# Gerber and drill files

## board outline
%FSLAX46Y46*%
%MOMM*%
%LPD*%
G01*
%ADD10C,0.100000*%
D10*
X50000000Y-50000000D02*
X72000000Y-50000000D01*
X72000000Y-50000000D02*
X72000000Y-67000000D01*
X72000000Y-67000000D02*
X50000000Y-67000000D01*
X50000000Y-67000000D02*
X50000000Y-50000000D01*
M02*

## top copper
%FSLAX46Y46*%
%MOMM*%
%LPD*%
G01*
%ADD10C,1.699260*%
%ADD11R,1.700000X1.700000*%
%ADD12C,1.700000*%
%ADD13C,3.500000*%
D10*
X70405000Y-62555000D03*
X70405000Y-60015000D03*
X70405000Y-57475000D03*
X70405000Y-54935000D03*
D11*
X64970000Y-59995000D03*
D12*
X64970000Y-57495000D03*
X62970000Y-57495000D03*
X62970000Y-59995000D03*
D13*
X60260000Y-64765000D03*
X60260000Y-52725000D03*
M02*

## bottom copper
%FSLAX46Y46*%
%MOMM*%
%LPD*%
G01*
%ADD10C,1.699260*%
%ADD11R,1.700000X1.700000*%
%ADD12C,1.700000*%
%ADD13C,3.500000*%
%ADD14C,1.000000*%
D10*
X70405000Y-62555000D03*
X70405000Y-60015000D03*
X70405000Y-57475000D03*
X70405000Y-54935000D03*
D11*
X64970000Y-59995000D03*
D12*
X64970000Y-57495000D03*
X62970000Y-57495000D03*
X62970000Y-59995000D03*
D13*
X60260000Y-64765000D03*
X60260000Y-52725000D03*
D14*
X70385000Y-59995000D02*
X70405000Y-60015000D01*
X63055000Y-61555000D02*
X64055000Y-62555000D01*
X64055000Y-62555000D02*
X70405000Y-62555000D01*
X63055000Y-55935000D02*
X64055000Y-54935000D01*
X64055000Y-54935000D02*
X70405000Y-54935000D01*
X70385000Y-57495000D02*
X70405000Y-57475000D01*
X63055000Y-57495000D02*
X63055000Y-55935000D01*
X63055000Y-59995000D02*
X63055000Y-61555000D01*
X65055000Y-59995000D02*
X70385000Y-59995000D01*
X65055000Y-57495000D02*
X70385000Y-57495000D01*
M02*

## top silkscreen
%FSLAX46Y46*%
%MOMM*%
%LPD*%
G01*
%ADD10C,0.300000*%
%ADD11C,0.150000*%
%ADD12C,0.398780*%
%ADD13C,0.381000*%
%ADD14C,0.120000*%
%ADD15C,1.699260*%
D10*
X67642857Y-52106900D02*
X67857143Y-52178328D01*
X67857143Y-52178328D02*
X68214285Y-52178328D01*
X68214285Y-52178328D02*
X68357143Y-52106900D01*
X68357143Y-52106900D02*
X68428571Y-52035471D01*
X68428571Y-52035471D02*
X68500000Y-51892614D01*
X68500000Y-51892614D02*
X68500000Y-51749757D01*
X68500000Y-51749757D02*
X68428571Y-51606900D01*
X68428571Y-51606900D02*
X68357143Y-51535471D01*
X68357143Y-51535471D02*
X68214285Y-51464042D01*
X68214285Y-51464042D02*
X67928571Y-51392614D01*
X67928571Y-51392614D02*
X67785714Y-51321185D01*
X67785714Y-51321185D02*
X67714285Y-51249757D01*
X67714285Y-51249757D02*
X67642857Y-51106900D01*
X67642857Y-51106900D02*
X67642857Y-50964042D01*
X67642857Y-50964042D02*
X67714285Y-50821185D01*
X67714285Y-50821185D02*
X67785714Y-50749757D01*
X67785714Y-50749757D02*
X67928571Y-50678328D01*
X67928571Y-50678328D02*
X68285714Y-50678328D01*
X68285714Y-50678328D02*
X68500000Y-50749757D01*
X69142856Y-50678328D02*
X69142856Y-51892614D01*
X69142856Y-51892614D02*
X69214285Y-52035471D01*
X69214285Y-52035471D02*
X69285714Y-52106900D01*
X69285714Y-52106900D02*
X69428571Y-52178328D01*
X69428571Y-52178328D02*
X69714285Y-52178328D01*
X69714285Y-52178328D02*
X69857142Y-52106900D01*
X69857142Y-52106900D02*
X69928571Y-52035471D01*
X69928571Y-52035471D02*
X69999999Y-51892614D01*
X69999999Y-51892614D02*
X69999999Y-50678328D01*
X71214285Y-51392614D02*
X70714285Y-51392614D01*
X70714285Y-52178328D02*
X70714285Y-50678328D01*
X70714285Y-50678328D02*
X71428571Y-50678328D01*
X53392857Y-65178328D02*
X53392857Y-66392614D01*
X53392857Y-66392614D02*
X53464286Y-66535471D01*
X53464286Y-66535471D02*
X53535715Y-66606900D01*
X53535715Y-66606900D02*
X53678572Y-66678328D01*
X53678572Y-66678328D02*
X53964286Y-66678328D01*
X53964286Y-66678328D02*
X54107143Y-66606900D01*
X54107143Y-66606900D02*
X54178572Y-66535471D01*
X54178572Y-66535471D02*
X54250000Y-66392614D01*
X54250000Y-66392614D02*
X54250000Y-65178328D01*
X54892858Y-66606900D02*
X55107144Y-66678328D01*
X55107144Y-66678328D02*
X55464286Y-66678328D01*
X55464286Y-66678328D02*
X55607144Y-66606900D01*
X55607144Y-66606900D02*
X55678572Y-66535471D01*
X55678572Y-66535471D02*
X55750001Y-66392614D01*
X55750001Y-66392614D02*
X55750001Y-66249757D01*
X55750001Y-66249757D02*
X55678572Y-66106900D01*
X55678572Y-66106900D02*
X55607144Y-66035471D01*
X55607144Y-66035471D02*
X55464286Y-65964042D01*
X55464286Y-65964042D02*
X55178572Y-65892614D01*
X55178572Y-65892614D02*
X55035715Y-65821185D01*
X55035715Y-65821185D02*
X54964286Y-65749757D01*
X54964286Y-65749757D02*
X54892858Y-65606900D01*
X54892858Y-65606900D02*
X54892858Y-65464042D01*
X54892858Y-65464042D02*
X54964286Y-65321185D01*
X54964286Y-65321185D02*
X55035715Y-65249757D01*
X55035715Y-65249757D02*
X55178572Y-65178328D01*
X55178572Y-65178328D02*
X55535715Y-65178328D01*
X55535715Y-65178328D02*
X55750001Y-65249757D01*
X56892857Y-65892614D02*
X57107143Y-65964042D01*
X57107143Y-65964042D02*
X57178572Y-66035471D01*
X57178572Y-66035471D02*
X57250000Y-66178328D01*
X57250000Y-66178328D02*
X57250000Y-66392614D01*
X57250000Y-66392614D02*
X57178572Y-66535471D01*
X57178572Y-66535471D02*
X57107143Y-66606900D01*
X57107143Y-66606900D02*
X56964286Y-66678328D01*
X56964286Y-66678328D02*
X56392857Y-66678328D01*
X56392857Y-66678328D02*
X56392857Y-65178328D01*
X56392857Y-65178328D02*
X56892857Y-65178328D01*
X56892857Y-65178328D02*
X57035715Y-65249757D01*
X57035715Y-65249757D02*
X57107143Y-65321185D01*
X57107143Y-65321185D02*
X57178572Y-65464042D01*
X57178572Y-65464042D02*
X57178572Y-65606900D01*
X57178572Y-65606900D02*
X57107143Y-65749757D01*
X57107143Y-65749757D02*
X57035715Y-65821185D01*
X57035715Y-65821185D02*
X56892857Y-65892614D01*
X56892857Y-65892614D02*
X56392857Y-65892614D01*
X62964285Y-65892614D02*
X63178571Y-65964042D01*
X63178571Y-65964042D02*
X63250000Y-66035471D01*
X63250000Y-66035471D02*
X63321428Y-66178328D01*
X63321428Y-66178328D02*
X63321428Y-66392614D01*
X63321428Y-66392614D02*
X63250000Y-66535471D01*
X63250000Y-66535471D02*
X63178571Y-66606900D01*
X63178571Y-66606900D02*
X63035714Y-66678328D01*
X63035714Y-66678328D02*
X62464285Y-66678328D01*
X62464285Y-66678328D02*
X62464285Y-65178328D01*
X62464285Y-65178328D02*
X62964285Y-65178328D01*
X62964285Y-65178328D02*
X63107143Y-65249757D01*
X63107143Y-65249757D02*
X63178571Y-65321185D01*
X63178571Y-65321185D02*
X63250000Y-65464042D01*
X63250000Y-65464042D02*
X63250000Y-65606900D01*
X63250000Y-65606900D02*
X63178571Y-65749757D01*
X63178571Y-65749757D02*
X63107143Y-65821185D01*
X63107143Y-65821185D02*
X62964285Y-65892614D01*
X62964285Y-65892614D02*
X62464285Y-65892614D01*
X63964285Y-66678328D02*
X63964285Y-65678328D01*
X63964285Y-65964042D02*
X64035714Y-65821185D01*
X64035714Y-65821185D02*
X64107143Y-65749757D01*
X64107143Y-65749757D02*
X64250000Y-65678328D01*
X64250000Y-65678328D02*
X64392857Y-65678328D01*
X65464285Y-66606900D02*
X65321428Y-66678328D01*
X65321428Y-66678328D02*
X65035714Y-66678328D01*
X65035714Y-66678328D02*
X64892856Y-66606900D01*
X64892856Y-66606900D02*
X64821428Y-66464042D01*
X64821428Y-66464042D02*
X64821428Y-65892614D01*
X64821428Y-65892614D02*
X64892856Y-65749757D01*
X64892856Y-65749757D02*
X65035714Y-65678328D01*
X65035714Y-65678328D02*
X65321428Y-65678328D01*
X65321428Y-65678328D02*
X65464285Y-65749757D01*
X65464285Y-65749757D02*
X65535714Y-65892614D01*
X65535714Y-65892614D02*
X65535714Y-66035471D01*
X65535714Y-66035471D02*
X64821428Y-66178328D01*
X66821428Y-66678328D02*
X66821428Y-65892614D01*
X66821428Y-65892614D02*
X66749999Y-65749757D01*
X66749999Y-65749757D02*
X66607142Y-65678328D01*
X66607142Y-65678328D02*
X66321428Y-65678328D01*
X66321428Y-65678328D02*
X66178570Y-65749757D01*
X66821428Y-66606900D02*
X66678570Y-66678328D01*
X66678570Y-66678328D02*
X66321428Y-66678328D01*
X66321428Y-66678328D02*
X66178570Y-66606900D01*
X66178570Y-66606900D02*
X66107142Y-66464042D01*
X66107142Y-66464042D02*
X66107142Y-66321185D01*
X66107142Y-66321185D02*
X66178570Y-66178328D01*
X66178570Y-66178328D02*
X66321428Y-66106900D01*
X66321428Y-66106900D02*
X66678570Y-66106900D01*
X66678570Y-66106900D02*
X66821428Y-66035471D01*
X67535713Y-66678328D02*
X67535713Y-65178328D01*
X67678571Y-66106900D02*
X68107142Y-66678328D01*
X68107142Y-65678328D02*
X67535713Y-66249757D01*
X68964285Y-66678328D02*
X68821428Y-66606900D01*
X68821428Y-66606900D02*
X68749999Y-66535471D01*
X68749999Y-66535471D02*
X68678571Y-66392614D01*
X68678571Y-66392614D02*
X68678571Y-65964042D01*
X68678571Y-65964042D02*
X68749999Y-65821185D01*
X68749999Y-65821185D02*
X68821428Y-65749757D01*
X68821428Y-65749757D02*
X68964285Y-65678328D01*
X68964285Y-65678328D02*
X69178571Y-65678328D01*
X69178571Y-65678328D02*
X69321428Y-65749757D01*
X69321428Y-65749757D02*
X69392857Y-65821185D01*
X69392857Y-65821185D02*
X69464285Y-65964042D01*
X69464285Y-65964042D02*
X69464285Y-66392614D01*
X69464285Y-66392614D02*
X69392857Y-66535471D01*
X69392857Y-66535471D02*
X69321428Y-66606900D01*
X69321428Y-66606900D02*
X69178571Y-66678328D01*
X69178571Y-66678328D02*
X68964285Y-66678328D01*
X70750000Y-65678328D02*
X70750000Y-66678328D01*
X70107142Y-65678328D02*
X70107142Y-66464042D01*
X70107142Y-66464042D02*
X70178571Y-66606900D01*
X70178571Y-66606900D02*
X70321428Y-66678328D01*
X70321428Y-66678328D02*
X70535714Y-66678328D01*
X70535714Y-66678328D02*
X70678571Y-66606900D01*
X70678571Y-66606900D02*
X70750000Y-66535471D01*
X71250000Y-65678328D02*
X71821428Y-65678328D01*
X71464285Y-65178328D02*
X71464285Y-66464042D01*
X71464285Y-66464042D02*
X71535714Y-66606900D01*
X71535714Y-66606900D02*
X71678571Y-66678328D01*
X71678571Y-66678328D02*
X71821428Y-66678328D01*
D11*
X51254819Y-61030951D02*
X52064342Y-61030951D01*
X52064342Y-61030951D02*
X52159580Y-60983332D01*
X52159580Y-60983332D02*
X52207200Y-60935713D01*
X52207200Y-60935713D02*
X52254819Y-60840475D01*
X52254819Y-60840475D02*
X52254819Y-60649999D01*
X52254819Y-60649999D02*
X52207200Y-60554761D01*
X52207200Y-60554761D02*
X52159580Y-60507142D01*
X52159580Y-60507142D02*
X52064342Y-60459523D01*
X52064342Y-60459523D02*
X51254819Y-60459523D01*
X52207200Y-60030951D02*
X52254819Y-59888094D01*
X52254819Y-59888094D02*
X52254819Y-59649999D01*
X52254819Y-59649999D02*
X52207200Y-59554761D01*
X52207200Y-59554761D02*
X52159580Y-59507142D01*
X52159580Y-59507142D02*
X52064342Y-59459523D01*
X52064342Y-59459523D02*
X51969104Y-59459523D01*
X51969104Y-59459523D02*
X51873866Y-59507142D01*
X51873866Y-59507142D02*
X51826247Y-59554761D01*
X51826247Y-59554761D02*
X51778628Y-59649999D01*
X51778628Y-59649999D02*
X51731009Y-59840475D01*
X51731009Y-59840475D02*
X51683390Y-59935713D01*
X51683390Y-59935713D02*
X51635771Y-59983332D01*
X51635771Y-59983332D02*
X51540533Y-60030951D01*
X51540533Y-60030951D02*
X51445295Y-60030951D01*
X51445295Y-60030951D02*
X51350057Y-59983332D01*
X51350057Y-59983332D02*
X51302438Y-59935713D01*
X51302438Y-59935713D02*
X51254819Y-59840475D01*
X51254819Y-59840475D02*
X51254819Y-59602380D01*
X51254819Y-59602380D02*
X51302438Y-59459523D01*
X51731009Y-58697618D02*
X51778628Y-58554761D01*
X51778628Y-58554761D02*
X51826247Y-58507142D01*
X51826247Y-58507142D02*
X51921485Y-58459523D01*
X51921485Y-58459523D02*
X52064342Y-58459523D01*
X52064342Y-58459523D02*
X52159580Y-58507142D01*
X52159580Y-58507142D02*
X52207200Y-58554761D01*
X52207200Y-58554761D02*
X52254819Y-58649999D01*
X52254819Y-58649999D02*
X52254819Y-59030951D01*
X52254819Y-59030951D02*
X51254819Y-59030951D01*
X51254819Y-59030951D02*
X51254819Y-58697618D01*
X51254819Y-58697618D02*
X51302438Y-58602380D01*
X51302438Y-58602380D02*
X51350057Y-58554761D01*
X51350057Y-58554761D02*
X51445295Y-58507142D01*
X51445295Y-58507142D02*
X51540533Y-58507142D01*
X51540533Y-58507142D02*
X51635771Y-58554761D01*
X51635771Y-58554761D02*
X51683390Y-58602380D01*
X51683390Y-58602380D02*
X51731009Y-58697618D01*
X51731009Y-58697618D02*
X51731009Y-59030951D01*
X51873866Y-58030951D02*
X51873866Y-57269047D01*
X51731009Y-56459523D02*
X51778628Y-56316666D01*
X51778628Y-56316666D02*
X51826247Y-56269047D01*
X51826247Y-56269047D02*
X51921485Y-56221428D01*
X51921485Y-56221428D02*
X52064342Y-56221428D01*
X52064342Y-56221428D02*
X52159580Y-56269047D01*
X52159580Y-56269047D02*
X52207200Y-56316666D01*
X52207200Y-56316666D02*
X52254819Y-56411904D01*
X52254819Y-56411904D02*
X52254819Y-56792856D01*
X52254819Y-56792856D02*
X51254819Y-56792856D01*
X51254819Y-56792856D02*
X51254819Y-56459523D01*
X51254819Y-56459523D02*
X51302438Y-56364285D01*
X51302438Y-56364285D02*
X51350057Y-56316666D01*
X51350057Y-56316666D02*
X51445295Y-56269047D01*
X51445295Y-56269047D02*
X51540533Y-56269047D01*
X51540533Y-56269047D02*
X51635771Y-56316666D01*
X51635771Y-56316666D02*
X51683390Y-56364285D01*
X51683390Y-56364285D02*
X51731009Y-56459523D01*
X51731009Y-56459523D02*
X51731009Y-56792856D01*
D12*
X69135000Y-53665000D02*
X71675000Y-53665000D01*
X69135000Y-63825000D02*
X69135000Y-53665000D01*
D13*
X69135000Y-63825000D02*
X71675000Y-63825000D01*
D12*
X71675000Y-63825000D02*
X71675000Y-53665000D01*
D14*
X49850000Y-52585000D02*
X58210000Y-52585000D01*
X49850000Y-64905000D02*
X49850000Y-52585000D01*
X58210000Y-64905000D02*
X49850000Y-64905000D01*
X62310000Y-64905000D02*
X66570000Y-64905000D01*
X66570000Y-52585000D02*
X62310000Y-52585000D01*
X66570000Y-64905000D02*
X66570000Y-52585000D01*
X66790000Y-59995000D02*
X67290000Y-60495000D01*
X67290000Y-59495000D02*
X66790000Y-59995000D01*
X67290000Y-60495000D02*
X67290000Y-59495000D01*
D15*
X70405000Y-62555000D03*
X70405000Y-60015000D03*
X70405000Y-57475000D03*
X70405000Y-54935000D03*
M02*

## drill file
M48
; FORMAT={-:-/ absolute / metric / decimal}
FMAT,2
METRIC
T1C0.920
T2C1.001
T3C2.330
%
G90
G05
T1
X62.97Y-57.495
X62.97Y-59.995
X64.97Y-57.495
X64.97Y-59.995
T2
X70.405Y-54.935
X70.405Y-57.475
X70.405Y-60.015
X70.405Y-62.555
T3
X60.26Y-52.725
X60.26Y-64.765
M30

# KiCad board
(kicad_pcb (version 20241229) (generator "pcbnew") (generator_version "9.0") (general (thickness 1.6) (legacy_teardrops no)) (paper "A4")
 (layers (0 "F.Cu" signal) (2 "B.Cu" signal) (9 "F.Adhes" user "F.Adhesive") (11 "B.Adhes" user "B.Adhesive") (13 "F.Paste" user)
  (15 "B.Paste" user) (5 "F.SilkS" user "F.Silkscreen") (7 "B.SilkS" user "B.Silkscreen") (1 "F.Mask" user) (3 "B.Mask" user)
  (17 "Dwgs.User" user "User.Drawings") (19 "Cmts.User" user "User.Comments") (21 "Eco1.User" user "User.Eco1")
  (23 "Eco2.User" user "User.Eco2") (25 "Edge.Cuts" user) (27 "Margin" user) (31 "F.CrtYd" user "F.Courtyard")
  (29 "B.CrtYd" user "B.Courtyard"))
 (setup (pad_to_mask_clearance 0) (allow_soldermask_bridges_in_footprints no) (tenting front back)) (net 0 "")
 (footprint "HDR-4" (layer "F.Cu") (at 70.405 58.745 90)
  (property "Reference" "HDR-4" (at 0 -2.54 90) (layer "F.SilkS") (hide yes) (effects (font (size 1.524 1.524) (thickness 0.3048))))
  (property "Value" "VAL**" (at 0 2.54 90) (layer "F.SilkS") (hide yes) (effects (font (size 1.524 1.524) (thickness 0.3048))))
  (fp_line (start 5.08 -1.27) (end 5.08 1.27) (stroke (width 0.39878) (type solid)) (layer "F.SilkS"))
  (fp_line (start -5.08 -1.27) (end 5.08 -1.27) (stroke (width 0.39878) (type solid)) (layer "F.SilkS"))
  (fp_line (start -5.08 -1.27) (end -5.08 1.27) (stroke (width 0.381) (type solid)) (layer "F.SilkS"))
  (fp_line (start -5.08 1.27) (end 5.08 1.27) (stroke (width 0.39878) (type solid)) (layer "F.SilkS"))
  (pad "1" thru_hole circle (at -3.81 0 90) (size 1.69926 1.69926) (drill 1.00076) (layers "*.Cu" "*.Mask" "F.SilkS")
   (remove_unused_layers no))
  (pad "2" thru_hole circle (at -1.27 0 90) (size 1.69926 1.69926) (drill 1.00076) (layers "*.Cu" "*.Mask" "F.SilkS")
   (remove_unused_layers no))
  (pad "3" thru_hole circle (at 1.27 0 90) (size 1.69926 1.69926) (drill 1.00076) (layers "*.Cu" "*.Mask" "F.SilkS")
   (remove_unused_layers no))
  (pad "4" thru_hole circle (at 3.81 0 90) (size 1.69926 1.69926) (drill 1.00076) (layers "*.Cu" "*.Mask" "F.SilkS")
   (remove_unused_layers no)))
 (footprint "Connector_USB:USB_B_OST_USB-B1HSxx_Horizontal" (layer "F.Cu") (at 64.97 59.995 180)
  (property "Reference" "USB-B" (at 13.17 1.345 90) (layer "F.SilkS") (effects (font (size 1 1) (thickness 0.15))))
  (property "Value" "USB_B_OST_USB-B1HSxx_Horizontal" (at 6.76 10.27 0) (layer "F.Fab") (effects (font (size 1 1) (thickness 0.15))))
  (fp_line (start 15.12 7.41) (end 6.76 7.41) (stroke (width 0.12) (type solid)) (layer "F.SilkS"))
  (fp_line (start 15.12 -4.91) (end 15.12 7.41) (stroke (width 0.12) (type solid)) (layer "F.SilkS"))
  (fp_line (start 6.76 -4.91) (end 15.12 -4.91) (stroke (width 0.12) (type solid)) (layer "F.SilkS"))
  (fp_line (start 2.66 -4.91) (end -1.6 -4.91) (stroke (width 0.12) (type solid)) (layer "F.SilkS"))
  (fp_line (start -1.6 7.41) (end 2.66 7.41) (stroke (width 0.12) (type solid)) (layer "F.SilkS"))
  (fp_line (start -1.6 -4.91) (end -1.6 7.41) (stroke (width 0.12) (type solid)) (layer "F.SilkS"))
  (fp_line (start -1.82 0) (end -2.32 -0.5) (stroke (width 0.12) (type solid)) (layer "F.SilkS"))
  (fp_line (start -2.32 0.5) (end -1.82 0) (stroke (width 0.12) (type solid)) (layer "F.SilkS"))
  (fp_line (start -2.32 -0.5) (end -2.32 0.5) (stroke (width 0.12) (type solid)) (layer "F.SilkS"))
  (pad "1" thru_hole rect (at 0 0 180) (size 1.7 1.7) (drill 0.92) (layers "*.Cu" "*.Mask") (remove_unused_layers no))
  (pad "2" thru_hole circle (at 0 2.5 180) (size 1.7 1.7) (drill 0.92) (layers "*.Cu" "*.Mask") (remove_unused_layers no))
  (pad "3" thru_hole circle (at 2 2.5 180) (size 1.7 1.7) (drill 0.92) (layers "*.Cu" "*.Mask") (remove_unused_layers no))
  (pad "4" thru_hole circle (at 2 0 180) (size 1.7 1.7) (drill 0.92) (layers "*.Cu" "*.Mask") (remove_unused_layers no))
  (pad "5" thru_hole circle (at 4.71 -4.77 180) (size 3.5 3.5) (drill 2.33) (layers "*.Cu" "*.Mask") (remove_unused_layers no))
  (pad "5" thru_hole circle (at 4.71 7.27 180) (size 3.5 3.5) (drill 2.33) (layers "*.Cu" "*.Mask") (remove_unused_layers no)))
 (gr_line (start 50 50) (end 72 50) (stroke (width 0.1) (type solid)) (layer "Edge.Cuts"))
 (gr_line (start 72 50) (end 72 67) (stroke (width 0.1) (type solid)) (layer "Edge.Cuts"))
 (gr_line (start 72 67) (end 50 67) (stroke (width 0.1) (type solid)) (layer "Edge.Cuts"))
 (gr_line (start 50 67) (end 50 50) (stroke (width 0.1) (type solid)) (layer "Edge.Cuts"))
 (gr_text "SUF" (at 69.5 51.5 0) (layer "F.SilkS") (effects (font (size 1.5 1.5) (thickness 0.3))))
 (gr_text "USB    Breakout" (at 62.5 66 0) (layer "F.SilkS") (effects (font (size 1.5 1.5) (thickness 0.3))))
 (segment (start 70.385 59.995) (end 70.405 60.015) (width 1) (layer "B.Cu") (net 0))
 (segment (start 63.055 61.555) (end 64.055 62.555) (width 1) (layer "B.Cu") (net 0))
 (segment (start 64.055 62.555) (end 70.405 62.555) (width 1) (layer "B.Cu") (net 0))
 (segment (start 63.055 55.935) (end 64.055 54.935) (width 1) (layer "B.Cu") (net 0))
 (segment (start 64.055 54.935) (end 70.405 54.935) (width 1) (layer "B.Cu") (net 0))
 (segment (start 70.385 57.495) (end 70.405 57.475) (width 1) (layer "B.Cu") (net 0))
 (segment (start 63.055 57.495) (end 63.055 55.935) (width 1) (layer "B.Cu") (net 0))
 (segment (start 63.055 59.995) (end 63.055 61.555) (width 1) (layer "B.Cu") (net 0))
 (segment (start 65.055 59.995) (end 70.385 59.995) (width 1) (layer "B.Cu") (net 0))
 (segment (start 65.055 57.495) (end 70.385 57.495) (width 1) (layer "B.Cu") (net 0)))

